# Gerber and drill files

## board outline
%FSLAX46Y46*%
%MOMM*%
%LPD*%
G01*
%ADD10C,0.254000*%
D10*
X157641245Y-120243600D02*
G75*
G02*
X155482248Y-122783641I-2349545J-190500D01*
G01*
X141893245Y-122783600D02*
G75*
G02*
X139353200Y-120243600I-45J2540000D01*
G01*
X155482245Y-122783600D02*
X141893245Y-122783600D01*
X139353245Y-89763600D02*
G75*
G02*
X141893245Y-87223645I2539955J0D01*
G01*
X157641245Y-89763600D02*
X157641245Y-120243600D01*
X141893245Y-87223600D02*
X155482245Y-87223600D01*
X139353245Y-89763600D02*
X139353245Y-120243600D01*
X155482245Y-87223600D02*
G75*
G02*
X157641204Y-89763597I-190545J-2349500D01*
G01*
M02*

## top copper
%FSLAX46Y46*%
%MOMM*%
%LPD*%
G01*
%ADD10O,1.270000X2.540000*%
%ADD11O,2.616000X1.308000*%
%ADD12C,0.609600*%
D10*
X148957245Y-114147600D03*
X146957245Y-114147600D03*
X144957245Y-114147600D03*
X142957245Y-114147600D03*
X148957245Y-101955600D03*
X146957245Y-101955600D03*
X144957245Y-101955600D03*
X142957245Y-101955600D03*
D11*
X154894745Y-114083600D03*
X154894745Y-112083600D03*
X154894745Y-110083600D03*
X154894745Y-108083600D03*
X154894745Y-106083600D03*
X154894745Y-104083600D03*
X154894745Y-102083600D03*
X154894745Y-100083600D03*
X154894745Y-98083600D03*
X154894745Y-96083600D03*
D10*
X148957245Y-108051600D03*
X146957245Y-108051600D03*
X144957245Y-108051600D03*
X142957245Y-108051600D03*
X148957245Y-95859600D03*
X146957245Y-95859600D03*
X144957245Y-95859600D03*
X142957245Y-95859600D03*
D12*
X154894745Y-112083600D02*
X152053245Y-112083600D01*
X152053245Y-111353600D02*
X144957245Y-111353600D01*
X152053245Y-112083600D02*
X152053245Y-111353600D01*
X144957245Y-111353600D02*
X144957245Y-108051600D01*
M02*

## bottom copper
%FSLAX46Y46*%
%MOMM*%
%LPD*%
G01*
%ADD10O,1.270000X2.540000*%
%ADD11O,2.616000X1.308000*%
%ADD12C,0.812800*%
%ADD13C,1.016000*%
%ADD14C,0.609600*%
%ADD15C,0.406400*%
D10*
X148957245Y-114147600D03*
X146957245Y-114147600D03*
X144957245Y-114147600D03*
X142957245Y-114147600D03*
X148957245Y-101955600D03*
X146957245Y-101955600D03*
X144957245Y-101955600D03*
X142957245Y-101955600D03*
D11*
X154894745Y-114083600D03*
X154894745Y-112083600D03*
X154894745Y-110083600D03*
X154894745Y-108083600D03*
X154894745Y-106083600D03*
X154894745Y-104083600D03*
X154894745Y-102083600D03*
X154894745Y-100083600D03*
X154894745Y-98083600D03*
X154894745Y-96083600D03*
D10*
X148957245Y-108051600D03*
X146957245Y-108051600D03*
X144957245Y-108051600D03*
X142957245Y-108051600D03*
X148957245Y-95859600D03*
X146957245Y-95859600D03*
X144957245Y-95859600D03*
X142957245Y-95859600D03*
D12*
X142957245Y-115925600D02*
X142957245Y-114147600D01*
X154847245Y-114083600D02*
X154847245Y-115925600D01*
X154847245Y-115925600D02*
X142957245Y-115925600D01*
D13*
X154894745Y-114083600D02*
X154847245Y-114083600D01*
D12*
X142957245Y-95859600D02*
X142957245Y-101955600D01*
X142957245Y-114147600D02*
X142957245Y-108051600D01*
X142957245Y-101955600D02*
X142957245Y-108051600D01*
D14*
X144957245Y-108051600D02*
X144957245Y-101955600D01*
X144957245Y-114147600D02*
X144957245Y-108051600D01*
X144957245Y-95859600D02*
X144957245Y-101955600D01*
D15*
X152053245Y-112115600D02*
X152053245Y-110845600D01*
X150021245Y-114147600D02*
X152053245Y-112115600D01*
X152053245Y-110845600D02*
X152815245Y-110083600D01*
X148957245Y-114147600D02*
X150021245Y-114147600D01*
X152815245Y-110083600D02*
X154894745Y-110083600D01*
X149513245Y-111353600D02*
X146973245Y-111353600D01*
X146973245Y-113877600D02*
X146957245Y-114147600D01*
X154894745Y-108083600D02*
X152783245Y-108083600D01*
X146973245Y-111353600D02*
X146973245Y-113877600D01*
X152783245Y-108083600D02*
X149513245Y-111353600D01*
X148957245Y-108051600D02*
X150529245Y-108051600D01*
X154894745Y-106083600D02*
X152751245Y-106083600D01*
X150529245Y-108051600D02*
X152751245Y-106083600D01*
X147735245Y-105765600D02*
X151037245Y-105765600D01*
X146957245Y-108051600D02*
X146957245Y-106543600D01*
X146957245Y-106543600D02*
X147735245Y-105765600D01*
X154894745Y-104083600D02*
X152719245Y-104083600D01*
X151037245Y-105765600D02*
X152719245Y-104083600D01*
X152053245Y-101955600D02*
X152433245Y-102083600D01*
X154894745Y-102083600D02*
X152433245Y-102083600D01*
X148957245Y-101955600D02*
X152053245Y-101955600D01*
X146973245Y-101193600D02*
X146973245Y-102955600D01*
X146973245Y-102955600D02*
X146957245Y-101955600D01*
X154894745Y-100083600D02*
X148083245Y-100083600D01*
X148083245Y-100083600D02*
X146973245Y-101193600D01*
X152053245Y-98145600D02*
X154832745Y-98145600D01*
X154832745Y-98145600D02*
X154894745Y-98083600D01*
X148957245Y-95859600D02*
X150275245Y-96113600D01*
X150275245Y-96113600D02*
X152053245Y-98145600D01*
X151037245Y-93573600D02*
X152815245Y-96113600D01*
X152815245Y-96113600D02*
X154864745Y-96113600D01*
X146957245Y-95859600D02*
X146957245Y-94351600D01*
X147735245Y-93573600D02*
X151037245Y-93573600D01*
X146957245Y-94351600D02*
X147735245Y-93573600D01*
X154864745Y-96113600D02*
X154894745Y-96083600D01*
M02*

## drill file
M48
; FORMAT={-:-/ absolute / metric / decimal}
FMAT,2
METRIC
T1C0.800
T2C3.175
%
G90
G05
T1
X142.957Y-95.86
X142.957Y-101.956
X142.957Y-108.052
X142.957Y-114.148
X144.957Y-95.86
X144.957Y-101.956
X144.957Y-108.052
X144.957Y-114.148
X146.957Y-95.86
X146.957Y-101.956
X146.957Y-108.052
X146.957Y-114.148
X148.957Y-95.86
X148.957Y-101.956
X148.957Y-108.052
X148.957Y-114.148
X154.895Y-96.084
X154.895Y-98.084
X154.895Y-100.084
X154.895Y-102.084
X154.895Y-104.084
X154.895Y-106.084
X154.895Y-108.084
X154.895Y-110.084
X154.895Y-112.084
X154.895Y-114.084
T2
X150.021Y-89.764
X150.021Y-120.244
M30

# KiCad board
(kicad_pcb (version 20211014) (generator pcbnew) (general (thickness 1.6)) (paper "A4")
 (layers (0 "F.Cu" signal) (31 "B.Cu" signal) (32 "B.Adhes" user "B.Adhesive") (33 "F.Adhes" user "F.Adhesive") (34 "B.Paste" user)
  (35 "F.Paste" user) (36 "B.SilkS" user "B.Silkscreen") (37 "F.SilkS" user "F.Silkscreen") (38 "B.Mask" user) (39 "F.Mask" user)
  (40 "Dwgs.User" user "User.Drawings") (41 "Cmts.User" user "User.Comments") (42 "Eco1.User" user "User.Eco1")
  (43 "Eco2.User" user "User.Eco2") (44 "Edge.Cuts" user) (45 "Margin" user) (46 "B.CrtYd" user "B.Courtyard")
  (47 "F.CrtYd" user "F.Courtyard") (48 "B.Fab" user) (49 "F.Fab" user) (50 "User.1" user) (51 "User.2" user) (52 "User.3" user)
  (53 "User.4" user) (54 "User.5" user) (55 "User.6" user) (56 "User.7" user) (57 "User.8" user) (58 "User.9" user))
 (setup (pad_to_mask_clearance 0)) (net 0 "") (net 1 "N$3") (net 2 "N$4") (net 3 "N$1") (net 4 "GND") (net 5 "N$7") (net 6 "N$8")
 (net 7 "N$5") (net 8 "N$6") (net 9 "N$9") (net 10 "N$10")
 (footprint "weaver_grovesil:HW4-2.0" (layer "F.Cu") (at 145.957245 114.1476 180)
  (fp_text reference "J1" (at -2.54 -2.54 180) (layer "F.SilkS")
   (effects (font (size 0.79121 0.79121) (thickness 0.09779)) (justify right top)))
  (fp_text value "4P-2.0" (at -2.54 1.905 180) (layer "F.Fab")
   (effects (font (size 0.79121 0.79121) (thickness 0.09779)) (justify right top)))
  (pad "1" thru_hole oval (at -3 0 270) (size 2.54 1.27) (drill 0.8) (layers *.Cu *.Mask) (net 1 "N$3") (solder_mask_margin 0.1016))
  (pad "2" thru_hole oval (at -1 0 270) (size 2.54 1.27) (drill 0.8) (layers *.Cu *.Mask) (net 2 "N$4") (solder_mask_margin 0.1016))
  (pad "3" thru_hole oval (at 1 0 270) (size 2.54 1.27) (drill 0.8) (layers *.Cu *.Mask) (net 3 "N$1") (solder_mask_margin 0.1016))
  (pad "4" thru_hole oval (at 3 0 270) (size 2.54 1.27) (drill 0.8) (layers *.Cu *.Mask) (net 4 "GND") (solder_mask_margin 0.1016)))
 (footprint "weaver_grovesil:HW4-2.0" (layer "F.Cu") (at 145.957245 101.9556 180)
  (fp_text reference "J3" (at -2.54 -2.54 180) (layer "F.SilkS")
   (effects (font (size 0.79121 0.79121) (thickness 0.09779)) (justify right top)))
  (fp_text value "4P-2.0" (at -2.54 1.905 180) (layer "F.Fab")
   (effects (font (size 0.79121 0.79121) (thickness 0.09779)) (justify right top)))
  (pad "1" thru_hole oval (at -3 0 270) (size 2.54 1.27) (drill 0.8) (layers *.Cu *.Mask) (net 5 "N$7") (solder_mask_margin 0.1016))
  (pad "2" thru_hole oval (at -1 0 270) (size 2.54 1.27) (drill 0.8) (layers *.Cu *.Mask) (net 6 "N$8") (solder_mask_margin 0.1016))
  (pad "3" thru_hole oval (at 1 0 270) (size 2.54 1.27) (drill 0.8) (layers *.Cu *.Mask) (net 3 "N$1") (solder_mask_margin 0.1016))
  (pad "4" thru_hole oval (at 3 0 270) (size 2.54 1.27) (drill 0.8) (layers *.Cu *.Mask) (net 4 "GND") (solder_mask_margin 0.1016)))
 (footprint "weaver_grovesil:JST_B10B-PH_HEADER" (layer "F.Cu") (at 154.847245 110.0836 -90)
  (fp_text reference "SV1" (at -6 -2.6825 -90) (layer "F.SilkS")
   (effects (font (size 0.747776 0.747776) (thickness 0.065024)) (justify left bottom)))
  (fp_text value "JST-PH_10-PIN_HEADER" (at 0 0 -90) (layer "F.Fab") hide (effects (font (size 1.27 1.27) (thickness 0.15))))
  (pad "P1" thru_hole oval (at 4 -0.0475) (size 2.616 1.308) (drill 0.8) (layers *.Cu *.Mask) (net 4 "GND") (solder_mask_margin 0.1016))
  (pad "P2" thru_hole oval (at 2 -0.0475) (size 2.616 1.308) (drill 0.8) (layers *.Cu *.Mask) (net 3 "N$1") (solder_mask_margin 0.1016))
  (pad "P3" thru_hole oval (at 0 -0.0475) (size 2.616 1.308) (drill 0.8) (layers *.Cu *.Mask) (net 1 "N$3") (solder_mask_margin 0.1016))
  (pad "P4" thru_hole oval (at -2 -0.0475) (size 2.616 1.308) (drill 0.8) (layers *.Cu *.Mask) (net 2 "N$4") (solder_mask_margin 0.1016))
  (pad "P5" thru_hole oval (at -4 -0.0475) (size 2.616 1.308) (drill 0.8) (layers *.Cu *.Mask) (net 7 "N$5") (solder_mask_margin 0.1016))
  (pad "P6" thru_hole oval (at -6 -0.0475) (size 2.616 1.308) (drill 0.8) (layers *.Cu *.Mask) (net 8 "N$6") (solder_mask_margin 0.1016))
  (pad "P7" thru_hole oval (at -8 -0.0475) (size 2.616 1.308) (drill 0.8) (layers *.Cu *.Mask) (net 5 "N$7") (solder_mask_margin 0.1016))
  (pad "P8" thru_hole oval (at -10 -0.0475) (size 2.616 1.308) (drill 0.8) (layers *.Cu *.Mask) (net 6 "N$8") (solder_mask_margin 0.1016))
  (pad "P9" thru_hole oval (at -12 -0.0475) (size 2.616 1.308) (drill 0.8) (layers *.Cu *.Mask) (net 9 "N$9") (solder_mask_margin 0.1016))
  (pad "P10" thru_hole oval (at -14 -0.0475) (size 2.616 1.308) (drill 0.8) (layers *.Cu *.Mask) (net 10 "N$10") (solder_mask_margin 0.1016)))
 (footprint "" (layer "F.Cu") (at 150.021245 120.2436)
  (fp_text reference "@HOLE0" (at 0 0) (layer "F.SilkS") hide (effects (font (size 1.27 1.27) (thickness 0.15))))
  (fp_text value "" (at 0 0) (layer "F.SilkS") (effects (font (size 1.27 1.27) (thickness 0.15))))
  (pad "" np_thru_hole circle (at 0 0) (size 3.175 3.175) (drill 3.175) (layers *.Cu *.Mask)))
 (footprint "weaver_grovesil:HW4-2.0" (layer "F.Cu") (at 145.957245 108.0516 180)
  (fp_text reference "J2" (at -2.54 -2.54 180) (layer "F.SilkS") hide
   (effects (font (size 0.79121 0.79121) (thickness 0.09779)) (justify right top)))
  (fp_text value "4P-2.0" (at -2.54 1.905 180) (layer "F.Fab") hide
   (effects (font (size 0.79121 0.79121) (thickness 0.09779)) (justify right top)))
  (pad "1" thru_hole oval (at -3 0 270) (size 2.54 1.27) (drill 0.8) (layers *.Cu *.Mask) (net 7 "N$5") (solder_mask_margin 0.1016))
  (pad "2" thru_hole oval (at -1 0 270) (size 2.54 1.27) (drill 0.8) (layers *.Cu *.Mask) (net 8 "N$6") (solder_mask_margin 0.1016))
  (pad "3" thru_hole oval (at 1 0 270) (size 2.54 1.27) (drill 0.8) (layers *.Cu *.Mask) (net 3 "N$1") (solder_mask_margin 0.1016))
  (pad "4" thru_hole oval (at 3 0 270) (size 2.54 1.27) (drill 0.8) (layers *.Cu *.Mask) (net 4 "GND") (solder_mask_margin 0.1016)))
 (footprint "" (layer "F.Cu") (at 150.021245 89.7636)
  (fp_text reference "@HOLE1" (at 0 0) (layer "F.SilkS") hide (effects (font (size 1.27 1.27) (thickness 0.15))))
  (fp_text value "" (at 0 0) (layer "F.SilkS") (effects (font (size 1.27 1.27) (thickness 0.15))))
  (pad "" np_thru_hole circle (at 0 0) (size 3.175 3.175) (drill 3.175) (layers *.Cu *.Mask)))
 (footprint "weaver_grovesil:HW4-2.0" (layer "F.Cu") (at 145.957245 95.8596 180)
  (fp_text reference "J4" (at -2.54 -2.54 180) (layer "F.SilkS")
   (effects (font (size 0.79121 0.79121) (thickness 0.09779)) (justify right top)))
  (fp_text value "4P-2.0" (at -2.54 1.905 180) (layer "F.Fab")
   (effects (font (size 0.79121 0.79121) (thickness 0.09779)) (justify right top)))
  (pad "1" thru_hole oval (at -3 0 270) (size 2.54 1.27) (drill 0.8) (layers *.Cu *.Mask) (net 9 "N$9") (solder_mask_margin 0.1016))
  (pad "2" thru_hole oval (at -1 0 270) (size 2.54 1.27) (drill 0.8) (layers *.Cu *.Mask) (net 10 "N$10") (solder_mask_margin 0.1016))
  (pad "3" thru_hole oval (at 1 0 270) (size 2.54 1.27) (drill 0.8) (layers *.Cu *.Mask) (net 3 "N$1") (solder_mask_margin 0.1016))
  (pad "4" thru_hole oval (at 3 0 270) (size 2.54 1.27) (drill 0.8) (layers *.Cu *.Mask) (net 4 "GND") (solder_mask_margin 0.1016)))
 (gr_arc (start 157.641245 120.2436) (mid 157.087796 121.960744) (end 155.482245 122.7836) (layer "Edge.Cuts") (width 0.254))
 (gr_arc (start 141.893245 122.7836) (mid 140.097194 122.039651) (end 139.353245 120.2436) (layer "Edge.Cuts") (width 0.254))
 (gr_line (start 155.482245 122.7836) (end 141.893245 122.7836) (layer "Edge.Cuts") (width 0.254))
 (gr_arc (start 139.353245 89.7636) (mid 140.097194 87.967549) (end 141.893245 87.2236) (layer "Edge.Cuts") (width 0.254))
 (gr_line (start 157.641245 89.7636) (end 157.641245 120.2436) (layer "Edge.Cuts") (width 0.254))
 (gr_line (start 141.893245 87.2236) (end 155.482245 87.2236) (layer "Edge.Cuts") (width 0.254))
 (gr_line (start 139.353245 89.7636) (end 139.353245 120.2436) (layer "Edge.Cuts") (width 0.254))
 (gr_arc (start 155.482245 87.2236) (mid 157.087796 88.046456) (end 157.641245 89.7636) (layer "Edge.Cuts") (width 0.254))
 (segment (start 142.957245 115.9256) (end 142.957245 114.1476) (width 0.8128) (layer "B.Cu") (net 4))
 (segment (start 154.847245 114.0836) (end 154.847245 115.9256) (width 0.8128) (layer "B.Cu") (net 4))
 (segment (start 154.847245 115.9256) (end 142.957245 115.9256) (width 0.8128) (layer "B.Cu") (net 4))
 (segment (start 154.894745 114.0836) (end 154.847245 114.0836) (width 1.016) (layer "B.Cu") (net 4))
 (segment (start 142.957245 95.8596) (end 142.957245 101.9556) (width 0.8128) (layer "B.Cu") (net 4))
 (segment (start 142.957245 114.1476) (end 142.957245 108.0516) (width 0.8128) (layer "B.Cu") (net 4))
 (segment (start 142.957245 101.9556) (end 142.957245 108.0516) (width 0.8128) (layer "B.Cu") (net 4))
 (segment (start 154.894745 112.0836) (end 152.053245 112.0836) (width 0.6096) (layer "F.Cu") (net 3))
 (segment (start 152.053245 111.3536) (end 144.957245 111.3536) (width 0.6096) (layer "F.Cu") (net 3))
 (segment (start 152.053245 112.0836) (end 152.053245 111.3536) (width 0.6096) (layer "F.Cu") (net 3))
 (segment (start 144.957245 111.3536) (end 144.957245 108.0516) (width 0.6096) (layer "F.Cu") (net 3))
 (segment (start 144.957245 108.0516) (end 144.957245 101.9556) (width 0.6096) (layer "B.Cu") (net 3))
 (segment (start 144.957245 114.1476) (end 144.957245 108.0516) (width 0.6096) (layer "B.Cu") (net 3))
 (segment (start 144.957245 95.8596) (end 144.957245 101.9556) (width 0.6096) (layer "B.Cu") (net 3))
 (segment (start 152.053245 112.1156) (end 152.053245 110.8456) (width 0.4064) (layer "B.Cu") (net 1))
 (segment (start 150.021245 114.1476) (end 152.053245 112.1156) (width 0.4064) (layer "B.Cu") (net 1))
 (segment (start 152.053245 110.8456) (end 152.815245 110.0836) (width 0.4064) (layer "B.Cu") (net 1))
 (segment (start 148.957245 114.1476) (end 150.021245 114.1476) (width 0.4064) (layer "B.Cu") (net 1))
 (segment (start 152.815245 110.0836) (end 154.894745 110.0836) (width 0.4064) (layer "B.Cu") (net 1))
 (segment (start 149.513245 111.3536) (end 146.973245 111.3536) (width 0.4064) (layer "B.Cu") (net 2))
 (segment (start 146.973245 113.8776) (end 146.957245 114.1476) (width 0.4064) (layer "B.Cu") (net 2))
 (segment (start 154.894745 108.0836) (end 152.783245 108.0836) (width 0.4064) (layer "B.Cu") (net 2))
 (segment (start 146.973245 111.3536) (end 146.973245 113.8776) (width 0.4064) (layer "B.Cu") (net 2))
 (segment (start 152.783245 108.0836) (end 149.513245 111.3536) (width 0.4064) (layer "B.Cu") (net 2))
 (segment (start 148.957245 108.0516) (end 150.529245 108.0516) (width 0.4064) (layer "B.Cu") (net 7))
 (segment (start 154.894745 106.0836) (end 152.751245 106.0836) (width 0.4064) (layer "B.Cu") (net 7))
 (segment (start 150.529245 108.0516) (end 152.751245 106.0836) (width 0.4064) (layer "B.Cu") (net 7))
 (segment (start 147.735245 105.7656) (end 151.037245 105.7656) (width 0.4064) (layer "B.Cu") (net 8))
 (segment (start 146.957245 108.0516) (end 146.957245 106.5436) (width 0.4064) (layer "B.Cu") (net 8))
 (segment (start 146.957245 106.5436) (end 147.735245 105.7656) (width 0.4064) (layer "B.Cu") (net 8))
 (segment (start 154.894745 104.0836) (end 152.719245 104.0836) (width 0.4064) (layer "B.Cu") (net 8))
 (segment (start 151.037245 105.7656) (end 152.719245 104.0836) (width 0.4064) (layer "B.Cu") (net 8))
 (segment (start 152.053245 101.9556) (end 152.433245 102.0836) (width 0.4064) (layer "B.Cu") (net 5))
 (segment (start 154.894745 102.0836) (end 152.433245 102.0836) (width 0.4064) (layer "B.Cu") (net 5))
 (segment (start 148.957245 101.9556) (end 152.053245 101.9556) (width 0.4064) (layer "B.Cu") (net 5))
 (segment (start 146.973245 101.1936) (end 146.973245 102.9556) (width 0.4064) (layer "B.Cu") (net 6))
 (segment (start 146.973245 102.9556) (end 146.957245 101.9556) (width 0.4064) (layer "B.Cu") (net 6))
 (segment (start 154.894745 100.0836) (end 148.083245 100.0836) (width 0.4064) (layer "B.Cu") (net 6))
 (segment (start 148.083245 100.0836) (end 146.973245 101.1936) (width 0.4064) (layer "B.Cu") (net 6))
 (segment (start 152.053245 98.1456) (end 154.832745 98.1456) (width 0.4064) (layer "B.Cu") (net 9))
 (segment (start 154.832745 98.1456) (end 154.894745 98.0836) (width 0.4064) (layer "B.Cu") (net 9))
 (segment (start 148.957245 95.8596) (end 150.275245 96.1136) (width 0.4064) (layer "B.Cu") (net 9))
 (segment (start 150.275245 96.1136) (end 152.053245 98.1456) (width 0.4064) (layer "B.Cu") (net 9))
 (segment (start 151.037245 93.5736) (end 152.815245 96.1136) (width 0.4064) (layer "B.Cu") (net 10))
 (segment (start 152.815245 96.1136) (end 154.864745 96.1136) (width 0.4064) (layer "B.Cu") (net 10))
 (segment (start 146.957245 95.8596) (end 146.957245 94.3516) (width 0.4064) (layer "B.Cu") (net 10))
 (segment (start 147.735245 93.5736) (end 151.037245 93.5736) (width 0.4064) (layer "B.Cu") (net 10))
 (segment (start 146.957245 94.3516) (end 147.735245 93.5736) (width 0.4064) (layer "B.Cu") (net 10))
 (segment (start 154.864745 96.1136) (end 154.894745 96.0836) (width 0.4064) (layer "B.Cu") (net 10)))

